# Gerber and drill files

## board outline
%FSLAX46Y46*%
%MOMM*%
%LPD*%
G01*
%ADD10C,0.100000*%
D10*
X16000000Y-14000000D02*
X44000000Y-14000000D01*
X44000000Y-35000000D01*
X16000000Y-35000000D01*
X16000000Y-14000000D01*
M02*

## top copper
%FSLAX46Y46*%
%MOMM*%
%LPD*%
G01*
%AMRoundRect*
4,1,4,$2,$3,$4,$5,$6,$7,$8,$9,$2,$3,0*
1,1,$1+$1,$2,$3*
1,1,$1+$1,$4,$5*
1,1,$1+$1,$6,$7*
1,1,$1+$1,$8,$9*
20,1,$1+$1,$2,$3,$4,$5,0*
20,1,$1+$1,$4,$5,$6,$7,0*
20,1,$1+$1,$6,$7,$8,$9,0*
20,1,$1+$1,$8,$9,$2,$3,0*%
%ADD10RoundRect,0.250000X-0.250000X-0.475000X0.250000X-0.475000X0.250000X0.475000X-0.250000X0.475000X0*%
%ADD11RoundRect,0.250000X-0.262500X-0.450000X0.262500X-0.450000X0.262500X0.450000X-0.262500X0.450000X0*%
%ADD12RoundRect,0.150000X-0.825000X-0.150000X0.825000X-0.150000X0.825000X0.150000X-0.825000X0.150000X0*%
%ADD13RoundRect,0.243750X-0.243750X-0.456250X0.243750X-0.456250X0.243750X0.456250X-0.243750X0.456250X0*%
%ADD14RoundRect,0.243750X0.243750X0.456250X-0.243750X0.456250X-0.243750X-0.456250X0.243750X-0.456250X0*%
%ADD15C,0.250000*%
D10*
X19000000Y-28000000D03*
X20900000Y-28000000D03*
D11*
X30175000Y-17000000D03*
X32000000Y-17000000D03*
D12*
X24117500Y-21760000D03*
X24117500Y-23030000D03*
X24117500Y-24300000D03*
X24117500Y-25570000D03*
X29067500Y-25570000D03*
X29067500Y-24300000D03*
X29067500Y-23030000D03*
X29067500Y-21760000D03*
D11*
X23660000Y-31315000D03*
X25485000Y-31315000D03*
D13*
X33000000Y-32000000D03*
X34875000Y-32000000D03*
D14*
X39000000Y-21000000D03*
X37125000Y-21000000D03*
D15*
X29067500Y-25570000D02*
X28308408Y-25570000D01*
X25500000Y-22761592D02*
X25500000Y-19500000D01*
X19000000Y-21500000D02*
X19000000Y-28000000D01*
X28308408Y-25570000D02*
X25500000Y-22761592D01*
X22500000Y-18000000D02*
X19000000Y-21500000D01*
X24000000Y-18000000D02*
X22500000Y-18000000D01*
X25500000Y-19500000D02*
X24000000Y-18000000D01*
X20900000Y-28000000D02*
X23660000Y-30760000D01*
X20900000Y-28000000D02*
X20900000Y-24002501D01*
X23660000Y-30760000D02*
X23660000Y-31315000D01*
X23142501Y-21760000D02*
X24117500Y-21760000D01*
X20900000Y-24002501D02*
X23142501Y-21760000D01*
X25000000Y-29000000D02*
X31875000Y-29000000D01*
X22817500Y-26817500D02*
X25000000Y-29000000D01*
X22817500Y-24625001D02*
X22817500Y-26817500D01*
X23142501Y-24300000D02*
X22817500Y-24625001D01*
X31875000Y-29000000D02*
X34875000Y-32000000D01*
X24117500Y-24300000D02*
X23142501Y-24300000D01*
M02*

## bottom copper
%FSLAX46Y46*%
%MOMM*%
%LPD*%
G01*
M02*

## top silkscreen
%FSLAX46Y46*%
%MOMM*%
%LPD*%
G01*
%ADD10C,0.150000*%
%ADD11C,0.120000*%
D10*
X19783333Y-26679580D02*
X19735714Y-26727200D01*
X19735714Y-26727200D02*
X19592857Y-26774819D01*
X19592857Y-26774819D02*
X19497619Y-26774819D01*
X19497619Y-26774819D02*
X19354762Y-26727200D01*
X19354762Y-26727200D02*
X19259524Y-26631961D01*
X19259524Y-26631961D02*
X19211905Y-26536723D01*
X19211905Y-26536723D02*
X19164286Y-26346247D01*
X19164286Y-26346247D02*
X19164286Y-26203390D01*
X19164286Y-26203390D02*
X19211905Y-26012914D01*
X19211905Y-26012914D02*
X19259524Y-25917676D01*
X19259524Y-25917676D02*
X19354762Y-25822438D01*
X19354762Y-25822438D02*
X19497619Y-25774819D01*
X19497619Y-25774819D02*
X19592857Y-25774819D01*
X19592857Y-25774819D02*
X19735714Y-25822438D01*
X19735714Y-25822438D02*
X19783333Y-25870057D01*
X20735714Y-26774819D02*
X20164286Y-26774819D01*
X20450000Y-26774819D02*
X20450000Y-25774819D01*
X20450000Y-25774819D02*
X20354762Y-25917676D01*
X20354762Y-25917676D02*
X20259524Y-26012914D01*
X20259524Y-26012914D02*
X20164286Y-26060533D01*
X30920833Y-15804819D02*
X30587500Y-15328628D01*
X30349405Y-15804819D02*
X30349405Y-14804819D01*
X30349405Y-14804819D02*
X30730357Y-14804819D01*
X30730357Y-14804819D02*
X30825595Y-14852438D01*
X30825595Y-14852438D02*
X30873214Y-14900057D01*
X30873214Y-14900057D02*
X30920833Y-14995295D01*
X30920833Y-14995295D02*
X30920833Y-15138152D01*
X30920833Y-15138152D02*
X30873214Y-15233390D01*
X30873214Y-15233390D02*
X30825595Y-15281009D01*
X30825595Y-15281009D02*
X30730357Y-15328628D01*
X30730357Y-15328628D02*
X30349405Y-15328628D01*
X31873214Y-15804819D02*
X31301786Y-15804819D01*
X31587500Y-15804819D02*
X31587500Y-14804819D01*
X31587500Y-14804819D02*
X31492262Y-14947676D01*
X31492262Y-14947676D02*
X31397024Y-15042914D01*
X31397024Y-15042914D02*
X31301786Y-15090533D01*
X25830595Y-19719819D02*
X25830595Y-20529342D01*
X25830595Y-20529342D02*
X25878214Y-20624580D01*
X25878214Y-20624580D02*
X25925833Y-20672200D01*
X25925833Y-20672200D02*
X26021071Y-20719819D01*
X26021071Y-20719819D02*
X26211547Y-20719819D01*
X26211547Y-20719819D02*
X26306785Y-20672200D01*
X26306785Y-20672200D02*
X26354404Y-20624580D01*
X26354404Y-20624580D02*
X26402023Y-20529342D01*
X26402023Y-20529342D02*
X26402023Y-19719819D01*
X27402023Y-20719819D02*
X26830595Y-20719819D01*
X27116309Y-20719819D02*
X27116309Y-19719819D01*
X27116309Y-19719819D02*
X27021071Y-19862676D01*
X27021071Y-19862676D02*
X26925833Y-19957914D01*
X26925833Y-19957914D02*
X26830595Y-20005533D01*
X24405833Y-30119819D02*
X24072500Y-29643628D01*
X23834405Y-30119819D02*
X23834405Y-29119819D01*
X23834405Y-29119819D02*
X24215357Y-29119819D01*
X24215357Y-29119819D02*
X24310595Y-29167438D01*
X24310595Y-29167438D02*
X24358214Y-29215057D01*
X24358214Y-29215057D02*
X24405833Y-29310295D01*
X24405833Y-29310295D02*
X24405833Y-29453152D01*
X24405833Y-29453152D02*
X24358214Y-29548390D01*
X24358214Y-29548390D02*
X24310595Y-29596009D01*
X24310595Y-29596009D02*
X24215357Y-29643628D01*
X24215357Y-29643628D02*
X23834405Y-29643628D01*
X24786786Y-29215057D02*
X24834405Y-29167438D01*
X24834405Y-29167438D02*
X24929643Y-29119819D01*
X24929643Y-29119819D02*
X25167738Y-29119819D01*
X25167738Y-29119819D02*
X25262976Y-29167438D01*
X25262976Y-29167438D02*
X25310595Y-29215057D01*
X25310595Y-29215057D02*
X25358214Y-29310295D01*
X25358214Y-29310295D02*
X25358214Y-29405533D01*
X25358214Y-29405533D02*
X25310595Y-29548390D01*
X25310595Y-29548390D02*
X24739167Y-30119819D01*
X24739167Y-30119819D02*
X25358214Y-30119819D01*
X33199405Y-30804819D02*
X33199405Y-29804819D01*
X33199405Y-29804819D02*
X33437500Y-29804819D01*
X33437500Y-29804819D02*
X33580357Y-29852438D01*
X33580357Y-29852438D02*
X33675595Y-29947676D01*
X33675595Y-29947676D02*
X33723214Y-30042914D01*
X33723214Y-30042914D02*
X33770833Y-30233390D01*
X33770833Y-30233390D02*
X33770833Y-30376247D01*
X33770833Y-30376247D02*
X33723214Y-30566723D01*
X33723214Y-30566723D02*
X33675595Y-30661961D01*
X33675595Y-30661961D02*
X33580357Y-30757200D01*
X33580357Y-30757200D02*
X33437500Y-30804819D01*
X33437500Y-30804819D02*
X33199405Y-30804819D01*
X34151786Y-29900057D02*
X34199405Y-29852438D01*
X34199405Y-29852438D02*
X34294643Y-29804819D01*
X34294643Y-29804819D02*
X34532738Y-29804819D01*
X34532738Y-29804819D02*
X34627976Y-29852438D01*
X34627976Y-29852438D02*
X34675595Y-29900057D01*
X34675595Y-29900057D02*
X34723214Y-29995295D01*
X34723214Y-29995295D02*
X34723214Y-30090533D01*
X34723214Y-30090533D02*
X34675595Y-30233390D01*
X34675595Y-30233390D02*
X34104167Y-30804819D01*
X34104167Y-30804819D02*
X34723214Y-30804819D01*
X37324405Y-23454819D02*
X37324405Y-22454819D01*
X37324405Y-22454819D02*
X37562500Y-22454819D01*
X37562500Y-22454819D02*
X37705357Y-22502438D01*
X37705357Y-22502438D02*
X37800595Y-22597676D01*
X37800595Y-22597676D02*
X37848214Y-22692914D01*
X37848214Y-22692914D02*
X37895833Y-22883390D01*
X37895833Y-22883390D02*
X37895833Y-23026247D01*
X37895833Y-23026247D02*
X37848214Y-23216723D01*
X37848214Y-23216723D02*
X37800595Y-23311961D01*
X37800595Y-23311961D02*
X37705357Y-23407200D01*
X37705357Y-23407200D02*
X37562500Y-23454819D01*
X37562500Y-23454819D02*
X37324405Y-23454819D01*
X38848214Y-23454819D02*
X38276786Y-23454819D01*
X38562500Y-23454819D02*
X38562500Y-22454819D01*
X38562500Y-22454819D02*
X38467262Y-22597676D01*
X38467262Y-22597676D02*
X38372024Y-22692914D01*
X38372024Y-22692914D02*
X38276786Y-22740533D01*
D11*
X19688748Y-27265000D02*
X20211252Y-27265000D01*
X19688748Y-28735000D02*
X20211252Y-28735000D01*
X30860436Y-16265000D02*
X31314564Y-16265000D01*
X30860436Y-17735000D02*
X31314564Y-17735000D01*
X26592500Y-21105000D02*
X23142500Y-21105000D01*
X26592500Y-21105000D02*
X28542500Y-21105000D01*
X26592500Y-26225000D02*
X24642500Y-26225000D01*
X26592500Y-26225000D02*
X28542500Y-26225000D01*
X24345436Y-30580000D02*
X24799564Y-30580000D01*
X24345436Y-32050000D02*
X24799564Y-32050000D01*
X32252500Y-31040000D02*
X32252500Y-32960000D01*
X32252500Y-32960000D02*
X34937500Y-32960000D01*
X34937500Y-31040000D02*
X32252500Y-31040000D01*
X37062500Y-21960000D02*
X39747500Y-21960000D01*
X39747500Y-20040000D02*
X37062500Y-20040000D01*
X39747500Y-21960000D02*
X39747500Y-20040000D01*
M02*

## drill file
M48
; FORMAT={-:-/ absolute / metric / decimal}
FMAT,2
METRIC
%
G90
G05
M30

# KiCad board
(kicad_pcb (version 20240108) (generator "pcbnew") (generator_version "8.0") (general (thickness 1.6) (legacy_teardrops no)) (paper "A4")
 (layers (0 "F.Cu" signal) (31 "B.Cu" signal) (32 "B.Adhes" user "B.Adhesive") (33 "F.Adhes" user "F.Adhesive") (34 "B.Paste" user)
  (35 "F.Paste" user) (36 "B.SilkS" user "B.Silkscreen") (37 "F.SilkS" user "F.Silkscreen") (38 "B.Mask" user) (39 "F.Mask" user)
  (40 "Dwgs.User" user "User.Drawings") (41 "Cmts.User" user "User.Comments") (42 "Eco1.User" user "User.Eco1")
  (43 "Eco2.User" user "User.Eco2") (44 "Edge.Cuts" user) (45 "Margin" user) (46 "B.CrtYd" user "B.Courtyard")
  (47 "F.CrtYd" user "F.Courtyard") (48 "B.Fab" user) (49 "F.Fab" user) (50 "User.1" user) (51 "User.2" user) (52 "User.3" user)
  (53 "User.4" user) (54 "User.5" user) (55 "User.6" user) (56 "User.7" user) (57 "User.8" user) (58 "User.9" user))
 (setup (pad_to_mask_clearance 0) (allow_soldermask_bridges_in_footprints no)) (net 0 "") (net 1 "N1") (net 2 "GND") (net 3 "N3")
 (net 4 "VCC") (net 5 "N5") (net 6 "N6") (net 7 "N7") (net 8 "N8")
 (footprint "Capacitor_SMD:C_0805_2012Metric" (layer "F.Cu") (at 19.95 28)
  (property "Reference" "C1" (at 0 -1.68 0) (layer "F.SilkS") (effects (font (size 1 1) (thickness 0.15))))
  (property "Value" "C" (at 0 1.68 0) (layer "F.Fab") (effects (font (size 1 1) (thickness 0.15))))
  (fp_line (start -0.261252 -0.735) (end 0.261252 -0.735) (stroke (width 0.12) (type solid)) (layer "F.SilkS"))
  (fp_line (start -0.261252 0.735) (end 0.261252 0.735) (stroke (width 0.12) (type solid)) (layer "F.SilkS"))
  (pad "1" smd roundrect (at -0.95 0) (size 1 1.45) (layers "F.Cu" "F.Paste" "F.Mask") (roundrect_rratio 0.25) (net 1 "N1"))
  (pad "2" smd roundrect (at 0.95 0) (size 1 1.45) (layers "F.Cu" "F.Paste" "F.Mask") (roundrect_rratio 0.25) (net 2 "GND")))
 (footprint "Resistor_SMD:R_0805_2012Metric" (layer "F.Cu") (at 31.0875 17)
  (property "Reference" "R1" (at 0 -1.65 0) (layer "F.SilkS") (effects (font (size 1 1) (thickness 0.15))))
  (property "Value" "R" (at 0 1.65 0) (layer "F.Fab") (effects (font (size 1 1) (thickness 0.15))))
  (fp_line (start -0.227064 -0.735) (end 0.227064 -0.735) (stroke (width 0.12) (type solid)) (layer "F.SilkS"))
  (fp_line (start -0.227064 0.735) (end 0.227064 0.735) (stroke (width 0.12) (type solid)) (layer "F.SilkS"))
  (pad "1" smd roundrect (at -0.9125 0) (size 1.025 1.4) (layers "F.Cu" "F.Paste" "F.Mask") (roundrect_rratio 0.243902) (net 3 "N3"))
  (pad "2" smd roundrect (at 0.9125 0) (size 1.025 1.4) (layers "F.Cu" "F.Paste" "F.Mask") (roundrect_rratio 0.243902) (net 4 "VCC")))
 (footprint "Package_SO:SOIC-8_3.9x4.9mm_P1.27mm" (layer "F.Cu") (at 26.5925 23.665)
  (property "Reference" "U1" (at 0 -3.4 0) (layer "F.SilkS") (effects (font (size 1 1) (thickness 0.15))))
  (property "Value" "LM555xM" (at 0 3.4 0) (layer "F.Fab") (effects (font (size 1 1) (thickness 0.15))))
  (fp_line (start 0 -2.56) (end -3.45 -2.56) (stroke (width 0.12) (type solid)) (layer "F.SilkS"))
  (fp_line (start 0 -2.56) (end 1.95 -2.56) (stroke (width 0.12) (type solid)) (layer "F.SilkS"))
  (fp_line (start 0 2.56) (end -1.95 2.56) (stroke (width 0.12) (type solid)) (layer "F.SilkS"))
  (fp_line (start 0 2.56) (end 1.95 2.56) (stroke (width 0.12) (type solid)) (layer "F.SilkS"))
  (pad "1" smd roundrect (at -2.475 -1.905) (size 1.95 0.6) (layers "F.Cu" "F.Paste" "F.Mask") (roundrect_rratio 0.25) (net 2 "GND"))
  (pad "2" smd roundrect (at -2.475 -0.635) (size 1.95 0.6) (layers "F.Cu" "F.Paste" "F.Mask") (roundrect_rratio 0.25) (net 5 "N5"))
  (pad "3" smd roundrect (at -2.475 0.635) (size 1.95 0.6) (layers "F.Cu" "F.Paste" "F.Mask") (roundrect_rratio 0.25) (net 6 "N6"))
  (pad "4" smd roundrect (at -2.475 1.905) (size 1.95 0.6) (layers "F.Cu" "F.Paste" "F.Mask") (roundrect_rratio 0.25) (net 4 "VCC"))
  (pad "5" smd roundrect (at 2.475 1.905) (size 1.95 0.6) (layers "F.Cu" "F.Paste" "F.Mask") (roundrect_rratio 0.25) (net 1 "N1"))
  (pad "6" smd roundrect (at 2.475 0.635) (size 1.95 0.6) (layers "F.Cu" "F.Paste" "F.Mask") (roundrect_rratio 0.25) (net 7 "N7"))
  (pad "7" smd roundrect (at 2.475 -0.635) (size 1.95 0.6) (layers "F.Cu" "F.Paste" "F.Mask") (roundrect_rratio 0.25) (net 7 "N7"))
  (pad "8" smd roundrect (at 2.475 -1.905) (size 1.95 0.6) (layers "F.Cu" "F.Paste" "F.Mask") (roundrect_rratio 0.25) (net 4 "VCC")))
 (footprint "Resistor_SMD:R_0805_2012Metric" (layer "F.Cu") (at 24.5725 31.315)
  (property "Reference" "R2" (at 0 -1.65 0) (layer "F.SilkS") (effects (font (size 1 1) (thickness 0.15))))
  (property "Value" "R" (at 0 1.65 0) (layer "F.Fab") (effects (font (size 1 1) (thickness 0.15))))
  (fp_line (start -0.227064 -0.735) (end 0.227064 -0.735) (stroke (width 0.12) (type solid)) (layer "F.SilkS"))
  (fp_line (start -0.227064 0.735) (end 0.227064 0.735) (stroke (width 0.12) (type solid)) (layer "F.SilkS"))
  (pad "1" smd roundrect (at -0.9125 0) (size 1.025 1.4) (layers "F.Cu" "F.Paste" "F.Mask") (roundrect_rratio 0.243902) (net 2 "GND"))
  (pad "2" smd roundrect (at 0.9125 0) (size 1.025 1.4) (layers "F.Cu" "F.Paste" "F.Mask") (roundrect_rratio 0.243902) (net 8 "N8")))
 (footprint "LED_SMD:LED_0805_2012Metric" (layer "F.Cu") (at 33.9375 32)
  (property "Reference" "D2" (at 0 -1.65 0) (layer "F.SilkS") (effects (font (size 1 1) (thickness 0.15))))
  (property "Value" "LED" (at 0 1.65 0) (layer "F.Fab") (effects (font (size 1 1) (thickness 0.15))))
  (fp_line (start -1.685 -0.96) (end -1.685 0.96) (stroke (width 0.12) (type solid)) (layer "F.SilkS"))
  (fp_line (start -1.685 0.96) (end 1 0.96) (stroke (width 0.12) (type solid)) (layer "F.SilkS"))
  (fp_line (start 1 -0.96) (end -1.685 -0.96) (stroke (width 0.12) (type solid)) (layer "F.SilkS"))
  (pad "1" smd roundrect (at -0.9375 0) (size 0.975 1.4) (layers "F.Cu" "F.Paste" "F.Mask") (roundrect_rratio 0.25) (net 8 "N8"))
  (pad "2" smd roundrect (at 0.9375 0) (size 0.975 1.4) (layers "F.Cu" "F.Paste" "F.Mask") (roundrect_rratio 0.25) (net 6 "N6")))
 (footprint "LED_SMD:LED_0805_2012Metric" (layer "F.Cu") (at 38.0625 21 180)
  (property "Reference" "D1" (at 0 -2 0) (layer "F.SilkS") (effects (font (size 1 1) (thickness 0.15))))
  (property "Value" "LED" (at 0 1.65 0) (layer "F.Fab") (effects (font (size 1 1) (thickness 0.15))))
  (fp_line (start 1 -0.96) (end -1.685 -0.96) (stroke (width 0.12) (type solid)) (layer "F.SilkS"))
  (fp_line (start -1.685 0.96) (end 1 0.96) (stroke (width 0.12) (type solid)) (layer "F.SilkS"))
  (fp_line (start -1.685 -0.96) (end -1.685 0.96) (stroke (width 0.12) (type solid)) (layer "F.SilkS"))
  (pad "1" smd roundrect (at -0.9375 0 180) (size 0.975 1.4) (layers "F.Cu" "F.Paste" "F.Mask") (roundrect_rratio 0.25) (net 6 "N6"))
  (pad "2" smd roundrect (at 0.9375 0 180) (size 0.975 1.4) (layers "F.Cu" "F.Paste" "F.Mask") (roundrect_rratio 0.25) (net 3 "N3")))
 (gr_rect (start 16 14) (end 44 35) (stroke (width 0.1) (type default)) (fill none) (layer "Edge.Cuts"))
 (segment (start 29.0675 25.57) (end 28.308408 25.57) (width 0.25) (layer "F.Cu") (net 1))
 (segment (start 25.5 22.761592) (end 25.5 19.5) (width 0.25) (layer "F.Cu") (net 1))
 (segment (start 19 21.5) (end 19 28) (width 0.25) (layer "F.Cu") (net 1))
 (segment (start 28.308408 25.57) (end 25.5 22.761592) (width 0.25) (layer "F.Cu") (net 1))
 (segment (start 22.5 18) (end 19 21.5) (width 0.25) (layer "F.Cu") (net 1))
 (segment (start 24 18) (end 22.5 18) (width 0.25) (layer "F.Cu") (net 1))
 (segment (start 25.5 19.5) (end 24 18) (width 0.25) (layer "F.Cu") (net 1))
 (segment (start 20.9 28) (end 23.66 30.76) (width 0.25) (layer "F.Cu") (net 2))
 (segment (start 20.9 28) (end 20.9 24.002501) (width 0.25) (layer "F.Cu") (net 2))
 (segment (start 23.66 30.76) (end 23.66 31.315) (width 0.25) (layer "F.Cu") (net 2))
 (segment (start 23.142501 21.76) (end 24.1175 21.76) (width 0.25) (layer "F.Cu") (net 2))
 (segment (start 20.9 24.002501) (end 23.142501 21.76) (width 0.25) (layer "F.Cu") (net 2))
 (segment (start 25 29) (end 31.875 29) (width 0.25) (layer "F.Cu") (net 6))
 (segment (start 22.8175 26.8175) (end 25 29) (width 0.25) (layer "F.Cu") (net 6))
 (segment (start 22.8175 24.625001) (end 22.8175 26.8175) (width 0.25) (layer "F.Cu") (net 6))
 (segment (start 23.142501 24.3) (end 22.8175 24.625001) (width 0.25) (layer "F.Cu") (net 6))
 (segment (start 31.875 29) (end 34.875 32) (width 0.25) (layer "F.Cu") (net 6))
 (segment (start 24.1175 24.3) (end 23.142501 24.3) (width 0.25) (layer "F.Cu") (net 6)))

